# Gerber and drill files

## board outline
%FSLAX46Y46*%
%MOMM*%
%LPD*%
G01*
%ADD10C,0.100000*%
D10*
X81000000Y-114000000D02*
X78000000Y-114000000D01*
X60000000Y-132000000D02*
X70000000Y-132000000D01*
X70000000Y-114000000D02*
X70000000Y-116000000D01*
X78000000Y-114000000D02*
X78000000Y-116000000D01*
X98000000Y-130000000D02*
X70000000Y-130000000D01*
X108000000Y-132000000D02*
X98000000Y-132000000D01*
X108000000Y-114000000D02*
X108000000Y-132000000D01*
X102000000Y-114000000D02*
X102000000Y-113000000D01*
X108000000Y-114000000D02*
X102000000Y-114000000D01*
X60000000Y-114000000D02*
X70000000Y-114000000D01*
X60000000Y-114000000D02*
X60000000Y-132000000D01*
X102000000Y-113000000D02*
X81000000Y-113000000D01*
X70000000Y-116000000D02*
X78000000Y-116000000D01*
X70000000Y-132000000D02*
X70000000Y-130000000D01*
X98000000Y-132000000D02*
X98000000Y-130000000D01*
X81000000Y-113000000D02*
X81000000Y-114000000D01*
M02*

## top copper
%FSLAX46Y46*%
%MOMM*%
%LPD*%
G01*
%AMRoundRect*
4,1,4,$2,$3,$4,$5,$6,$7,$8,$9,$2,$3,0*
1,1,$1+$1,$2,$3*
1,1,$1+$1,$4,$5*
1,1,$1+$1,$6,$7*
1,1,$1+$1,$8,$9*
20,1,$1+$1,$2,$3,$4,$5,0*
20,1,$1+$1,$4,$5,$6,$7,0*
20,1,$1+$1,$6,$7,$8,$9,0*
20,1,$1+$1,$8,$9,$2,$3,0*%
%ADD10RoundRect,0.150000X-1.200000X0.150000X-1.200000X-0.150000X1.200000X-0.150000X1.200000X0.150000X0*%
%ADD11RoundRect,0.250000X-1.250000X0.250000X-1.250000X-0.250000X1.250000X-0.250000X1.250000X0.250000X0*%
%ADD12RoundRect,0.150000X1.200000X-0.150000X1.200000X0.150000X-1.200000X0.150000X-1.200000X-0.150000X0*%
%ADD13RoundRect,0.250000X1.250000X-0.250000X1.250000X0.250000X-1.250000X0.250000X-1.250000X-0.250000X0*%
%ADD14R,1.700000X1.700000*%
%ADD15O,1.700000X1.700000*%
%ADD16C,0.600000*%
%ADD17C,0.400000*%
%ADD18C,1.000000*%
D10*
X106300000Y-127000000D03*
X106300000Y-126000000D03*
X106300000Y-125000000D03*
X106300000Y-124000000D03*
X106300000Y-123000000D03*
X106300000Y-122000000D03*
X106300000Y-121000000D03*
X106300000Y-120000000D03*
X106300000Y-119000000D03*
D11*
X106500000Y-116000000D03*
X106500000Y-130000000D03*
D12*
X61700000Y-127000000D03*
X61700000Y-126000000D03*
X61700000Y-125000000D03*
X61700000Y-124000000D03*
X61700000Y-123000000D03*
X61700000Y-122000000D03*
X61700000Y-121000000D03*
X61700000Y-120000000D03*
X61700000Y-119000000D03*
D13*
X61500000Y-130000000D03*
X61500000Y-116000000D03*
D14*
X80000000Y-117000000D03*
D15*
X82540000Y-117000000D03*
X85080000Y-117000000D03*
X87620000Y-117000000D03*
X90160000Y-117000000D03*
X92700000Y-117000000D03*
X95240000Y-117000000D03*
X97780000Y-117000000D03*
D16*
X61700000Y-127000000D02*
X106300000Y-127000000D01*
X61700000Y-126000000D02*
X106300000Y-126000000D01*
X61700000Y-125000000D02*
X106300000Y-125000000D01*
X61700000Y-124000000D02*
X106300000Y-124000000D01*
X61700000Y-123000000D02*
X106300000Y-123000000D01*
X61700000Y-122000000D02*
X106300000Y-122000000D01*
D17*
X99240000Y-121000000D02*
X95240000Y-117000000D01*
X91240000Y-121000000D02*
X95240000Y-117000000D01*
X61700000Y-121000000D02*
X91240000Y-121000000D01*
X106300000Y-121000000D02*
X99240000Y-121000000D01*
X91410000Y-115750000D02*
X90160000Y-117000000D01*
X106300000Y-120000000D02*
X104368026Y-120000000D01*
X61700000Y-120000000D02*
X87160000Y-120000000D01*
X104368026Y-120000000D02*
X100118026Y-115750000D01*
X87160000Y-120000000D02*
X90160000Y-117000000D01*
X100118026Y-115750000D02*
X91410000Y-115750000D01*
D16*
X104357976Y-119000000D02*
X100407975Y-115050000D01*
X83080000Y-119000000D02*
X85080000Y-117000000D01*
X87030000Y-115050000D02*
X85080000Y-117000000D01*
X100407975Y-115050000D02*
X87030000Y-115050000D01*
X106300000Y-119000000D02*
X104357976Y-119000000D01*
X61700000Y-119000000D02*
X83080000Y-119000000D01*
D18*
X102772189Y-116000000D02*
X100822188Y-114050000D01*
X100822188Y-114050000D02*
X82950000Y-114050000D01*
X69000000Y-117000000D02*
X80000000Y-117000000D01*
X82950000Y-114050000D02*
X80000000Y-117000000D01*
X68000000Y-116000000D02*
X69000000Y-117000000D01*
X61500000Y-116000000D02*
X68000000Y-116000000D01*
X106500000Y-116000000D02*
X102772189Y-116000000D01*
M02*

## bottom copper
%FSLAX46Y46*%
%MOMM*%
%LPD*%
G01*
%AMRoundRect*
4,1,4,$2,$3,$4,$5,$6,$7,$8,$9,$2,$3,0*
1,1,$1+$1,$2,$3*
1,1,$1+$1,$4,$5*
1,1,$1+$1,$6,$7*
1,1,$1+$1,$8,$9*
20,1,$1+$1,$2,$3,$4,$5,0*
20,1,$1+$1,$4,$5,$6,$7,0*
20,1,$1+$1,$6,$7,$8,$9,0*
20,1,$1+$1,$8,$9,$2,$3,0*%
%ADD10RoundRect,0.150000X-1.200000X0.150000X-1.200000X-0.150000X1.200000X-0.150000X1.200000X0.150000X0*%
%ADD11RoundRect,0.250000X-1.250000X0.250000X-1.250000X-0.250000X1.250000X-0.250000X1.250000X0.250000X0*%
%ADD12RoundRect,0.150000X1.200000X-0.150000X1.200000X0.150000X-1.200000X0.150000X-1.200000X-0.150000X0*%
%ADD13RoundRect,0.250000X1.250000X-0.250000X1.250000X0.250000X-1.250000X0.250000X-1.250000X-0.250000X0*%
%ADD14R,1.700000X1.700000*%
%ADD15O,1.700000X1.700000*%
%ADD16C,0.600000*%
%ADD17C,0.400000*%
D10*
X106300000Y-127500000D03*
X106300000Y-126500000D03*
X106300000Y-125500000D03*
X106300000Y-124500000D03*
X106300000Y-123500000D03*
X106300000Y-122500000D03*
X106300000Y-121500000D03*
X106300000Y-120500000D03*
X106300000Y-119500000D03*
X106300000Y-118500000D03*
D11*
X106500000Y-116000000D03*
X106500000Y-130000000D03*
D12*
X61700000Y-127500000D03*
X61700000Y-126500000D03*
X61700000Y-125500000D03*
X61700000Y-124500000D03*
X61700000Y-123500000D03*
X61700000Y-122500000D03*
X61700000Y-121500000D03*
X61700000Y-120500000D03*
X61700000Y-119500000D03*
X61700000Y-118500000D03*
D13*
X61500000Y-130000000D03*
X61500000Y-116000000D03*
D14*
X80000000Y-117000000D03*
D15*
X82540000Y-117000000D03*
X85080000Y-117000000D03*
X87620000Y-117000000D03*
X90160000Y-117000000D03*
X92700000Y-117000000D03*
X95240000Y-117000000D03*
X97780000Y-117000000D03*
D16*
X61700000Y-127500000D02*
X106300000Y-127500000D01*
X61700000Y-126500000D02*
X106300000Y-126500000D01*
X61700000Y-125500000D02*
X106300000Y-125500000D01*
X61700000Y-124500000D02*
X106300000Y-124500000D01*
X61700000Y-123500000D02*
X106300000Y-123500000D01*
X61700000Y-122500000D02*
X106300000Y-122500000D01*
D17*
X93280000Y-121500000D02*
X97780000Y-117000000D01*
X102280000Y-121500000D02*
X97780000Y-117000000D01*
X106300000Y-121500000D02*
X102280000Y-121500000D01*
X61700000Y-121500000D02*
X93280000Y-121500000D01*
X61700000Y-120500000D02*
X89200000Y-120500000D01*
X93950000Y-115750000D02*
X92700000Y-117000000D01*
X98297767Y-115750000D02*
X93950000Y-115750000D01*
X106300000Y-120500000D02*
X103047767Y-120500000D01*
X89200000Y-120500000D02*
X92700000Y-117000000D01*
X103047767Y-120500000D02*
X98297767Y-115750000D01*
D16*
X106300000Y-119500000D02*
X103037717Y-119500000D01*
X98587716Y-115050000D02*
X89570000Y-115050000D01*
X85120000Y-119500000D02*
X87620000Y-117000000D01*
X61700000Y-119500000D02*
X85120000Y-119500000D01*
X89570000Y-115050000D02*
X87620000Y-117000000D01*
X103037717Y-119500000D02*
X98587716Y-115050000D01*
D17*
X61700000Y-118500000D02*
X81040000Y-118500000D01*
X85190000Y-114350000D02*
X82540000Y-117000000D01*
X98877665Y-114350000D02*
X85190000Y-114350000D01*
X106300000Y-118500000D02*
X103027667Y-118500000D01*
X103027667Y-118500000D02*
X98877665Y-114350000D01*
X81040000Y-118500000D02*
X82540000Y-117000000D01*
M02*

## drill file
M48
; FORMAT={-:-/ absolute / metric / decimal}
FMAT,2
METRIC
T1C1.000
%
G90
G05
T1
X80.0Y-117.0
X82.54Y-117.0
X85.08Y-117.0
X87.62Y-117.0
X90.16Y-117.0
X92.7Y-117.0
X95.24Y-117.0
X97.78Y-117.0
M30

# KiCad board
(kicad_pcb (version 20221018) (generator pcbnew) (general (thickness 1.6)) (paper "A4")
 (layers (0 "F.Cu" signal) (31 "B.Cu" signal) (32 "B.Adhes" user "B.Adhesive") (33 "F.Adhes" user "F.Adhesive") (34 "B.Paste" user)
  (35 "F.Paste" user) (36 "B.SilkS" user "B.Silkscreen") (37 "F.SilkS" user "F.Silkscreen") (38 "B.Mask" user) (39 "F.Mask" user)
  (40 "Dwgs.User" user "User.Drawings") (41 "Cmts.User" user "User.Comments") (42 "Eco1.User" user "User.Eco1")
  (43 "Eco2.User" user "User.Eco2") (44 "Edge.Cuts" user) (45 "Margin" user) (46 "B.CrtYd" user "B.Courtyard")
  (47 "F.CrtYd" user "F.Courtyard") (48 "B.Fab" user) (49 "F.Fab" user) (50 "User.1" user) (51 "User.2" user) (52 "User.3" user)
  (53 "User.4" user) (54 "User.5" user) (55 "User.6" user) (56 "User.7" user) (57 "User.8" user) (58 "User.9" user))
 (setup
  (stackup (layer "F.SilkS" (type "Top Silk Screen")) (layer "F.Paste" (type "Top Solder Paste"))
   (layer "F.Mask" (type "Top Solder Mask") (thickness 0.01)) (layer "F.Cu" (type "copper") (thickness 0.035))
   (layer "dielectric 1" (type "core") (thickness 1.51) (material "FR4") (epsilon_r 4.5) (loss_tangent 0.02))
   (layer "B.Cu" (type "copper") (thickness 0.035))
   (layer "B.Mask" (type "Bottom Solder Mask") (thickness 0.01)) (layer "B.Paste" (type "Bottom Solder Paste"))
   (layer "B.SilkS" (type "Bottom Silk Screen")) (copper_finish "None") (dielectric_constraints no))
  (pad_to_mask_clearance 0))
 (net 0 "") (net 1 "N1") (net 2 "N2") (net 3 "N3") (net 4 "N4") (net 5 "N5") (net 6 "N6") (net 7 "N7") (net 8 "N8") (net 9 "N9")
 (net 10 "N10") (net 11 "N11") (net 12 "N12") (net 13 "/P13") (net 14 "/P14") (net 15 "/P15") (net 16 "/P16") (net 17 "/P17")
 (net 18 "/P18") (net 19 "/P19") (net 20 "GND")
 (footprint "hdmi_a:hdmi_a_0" (layer "F.Cu") (at 108 123 -90)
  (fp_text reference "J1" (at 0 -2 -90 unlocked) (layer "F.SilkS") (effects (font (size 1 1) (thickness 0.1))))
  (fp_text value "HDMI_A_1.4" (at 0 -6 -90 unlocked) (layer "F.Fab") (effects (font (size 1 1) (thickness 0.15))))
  (pad "1" smd roundrect (at 4.5 1.7 270) (size 0.6 2.7) (layers "B.Cu" "B.Paste" "B.Mask") (roundrect_rratio 0.25) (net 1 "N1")
   (thermal_bridge_angle 45))
  (pad "2" smd roundrect (at 4 1.7 270) (size 0.6 2.7) (layers "F.Cu" "F.Paste" "F.Mask") (roundrect_rratio 0.25) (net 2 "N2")
   (thermal_bridge_angle 45))
  (pad "3" smd roundrect (at 3.5 1.7 270) (size 0.6 2.7) (layers "B.Cu" "B.Paste" "B.Mask") (roundrect_rratio 0.25) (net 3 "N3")
   (thermal_bridge_angle 45))
  (pad "4" smd roundrect (at 3 1.7 270) (size 0.6 2.7) (layers "F.Cu" "F.Paste" "F.Mask") (roundrect_rratio 0.25) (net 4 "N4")
   (thermal_bridge_angle 45))
  (pad "5" smd roundrect (at 2.5 1.7 270) (size 0.6 2.7) (layers "B.Cu" "B.Paste" "B.Mask") (roundrect_rratio 0.25) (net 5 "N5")
   (thermal_bridge_angle 45))
  (pad "6" smd roundrect (at 2 1.7 270) (size 0.6 2.7) (layers "F.Cu" "F.Paste" "F.Mask") (roundrect_rratio 0.25) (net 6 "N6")
   (thermal_bridge_angle 45))
  (pad "7" smd roundrect (at 1.5 1.7 270) (size 0.6 2.7) (layers "B.Cu" "B.Paste" "B.Mask") (roundrect_rratio 0.25) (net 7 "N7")
   (thermal_bridge_angle 45))
  (pad "8" smd roundrect (at 1 1.7 270) (size 0.6 2.7) (layers "F.Cu" "F.Paste" "F.Mask") (roundrect_rratio 0.25) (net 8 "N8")
   (thermal_bridge_angle 45))
  (pad "9" smd roundrect (at 0.5 1.7 270) (size 0.6 2.7) (layers "B.Cu" "B.Paste" "B.Mask") (roundrect_rratio 0.25) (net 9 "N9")
   (thermal_bridge_angle 45))
  (pad "10" smd roundrect (at 0 1.7 270) (size 0.6 2.7) (layers "F.Cu" "F.Paste" "F.Mask") (roundrect_rratio 0.25) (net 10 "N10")
   (thermal_bridge_angle 45))
  (pad "11" smd roundrect (at -0.5 1.7 270) (size 0.6 2.7) (layers "B.Cu" "B.Paste" "B.Mask") (roundrect_rratio 0.25) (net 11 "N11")
   (thermal_bridge_angle 45))
  (pad "12" smd roundrect (at -1 1.7 270) (size 0.6 2.7) (layers "F.Cu" "F.Paste" "F.Mask") (roundrect_rratio 0.25) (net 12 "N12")
   (thermal_bridge_angle 45))
  (pad "13" smd roundrect (at -1.5 1.7 270) (size 0.6 2.7) (layers "B.Cu" "B.Paste" "B.Mask") (roundrect_rratio 0.25) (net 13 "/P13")
   (thermal_bridge_angle 45))
  (pad "14" smd roundrect (at -2 1.7 270) (size 0.6 2.7) (layers "F.Cu" "F.Paste" "F.Mask") (roundrect_rratio 0.25) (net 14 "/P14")
   (thermal_bridge_angle 45))
  (pad "15" smd roundrect (at -2.5 1.7 270) (size 0.6 2.7) (layers "B.Cu" "B.Paste" "B.Mask") (roundrect_rratio 0.25) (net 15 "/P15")
   (thermal_bridge_angle 45))
  (pad "16" smd roundrect (at -3 1.7 270) (size 0.6 2.7) (layers "F.Cu" "F.Paste" "F.Mask") (roundrect_rratio 0.25) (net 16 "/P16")
   (thermal_bridge_angle 45))
  (pad "17" smd roundrect (at -3.5 1.7 270) (size 0.6 2.7) (layers "B.Cu" "B.Paste" "B.Mask") (roundrect_rratio 0.25) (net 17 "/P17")
   (thermal_bridge_angle 45))
  (pad "18" smd roundrect (at -4 1.7 270) (size 0.6 2.7) (layers "F.Cu" "F.Paste" "F.Mask") (roundrect_rratio 0.25) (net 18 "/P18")
   (thermal_bridge_angle 45))
  (pad "19" smd roundrect (at -4.5 1.7 270) (size 0.6 2.7) (layers "B.Cu" "B.Paste" "B.Mask") (roundrect_rratio 0.25) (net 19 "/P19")
   (thermal_bridge_angle 45))
  (pad "SH" smd roundrect (at -7 1.5 270) (size 1 3) (layers "F.Cu" "F.Paste" "F.Mask") (roundrect_rratio 0.25) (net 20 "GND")
   (thermal_bridge_angle 45))
  (pad "SH" smd roundrect (at -7 1.5 270) (size 1 3) (layers "B.Cu" "B.Paste" "B.Mask") (roundrect_rratio 0.25) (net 20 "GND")
   (thermal_bridge_angle 45))
  (pad "SH" smd roundrect (at 7 1.5 270) (size 1 3) (layers "F.Cu" "F.Paste" "F.Mask") (roundrect_rratio 0.25) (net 20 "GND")
   (thermal_bridge_angle 45))
  (pad "SH" smd roundrect (at 7 1.5 270) (size 1 3) (layers "B.Cu" "B.Paste" "B.Mask") (roundrect_rratio 0.25) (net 20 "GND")
   (thermal_bridge_angle 45)))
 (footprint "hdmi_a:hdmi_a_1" (layer "F.Cu") (at 60 123 90)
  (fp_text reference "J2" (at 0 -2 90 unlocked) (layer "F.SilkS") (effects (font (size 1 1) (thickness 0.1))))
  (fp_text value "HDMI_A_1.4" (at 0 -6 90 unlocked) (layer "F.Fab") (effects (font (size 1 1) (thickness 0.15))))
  (pad "1" smd roundrect (at -4.5 1.7 90) (size 0.6 2.7) (layers "B.Cu" "B.Paste" "B.Mask") (roundrect_rratio 0.25) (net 1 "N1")
   (thermal_bridge_angle 45))
  (pad "2" smd roundrect (at -4 1.7 90) (size 0.6 2.7) (layers "F.Cu" "F.Paste" "F.Mask") (roundrect_rratio 0.25) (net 2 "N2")
   (thermal_bridge_angle 45))
  (pad "3" smd roundrect (at -3.5 1.7 90) (size 0.6 2.7) (layers "B.Cu" "B.Paste" "B.Mask") (roundrect_rratio 0.25) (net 3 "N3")
   (thermal_bridge_angle 45))
  (pad "4" smd roundrect (at -3 1.7 90) (size 0.6 2.7) (layers "F.Cu" "F.Paste" "F.Mask") (roundrect_rratio 0.25) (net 4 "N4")
   (thermal_bridge_angle 45))
  (pad "5" smd roundrect (at -2.5 1.7 90) (size 0.6 2.7) (layers "B.Cu" "B.Paste" "B.Mask") (roundrect_rratio 0.25) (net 5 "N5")
   (thermal_bridge_angle 45))
  (pad "6" smd roundrect (at -2 1.7 90) (size 0.6 2.7) (layers "F.Cu" "F.Paste" "F.Mask") (roundrect_rratio 0.25) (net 6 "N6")
   (thermal_bridge_angle 45))
  (pad "7" smd roundrect (at -1.5 1.7 90) (size 0.6 2.7) (layers "B.Cu" "B.Paste" "B.Mask") (roundrect_rratio 0.25) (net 7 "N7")
   (thermal_bridge_angle 45))
  (pad "8" smd roundrect (at -1 1.7 90) (size 0.6 2.7) (layers "F.Cu" "F.Paste" "F.Mask") (roundrect_rratio 0.25) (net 8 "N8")
   (thermal_bridge_angle 45))
  (pad "9" smd roundrect (at -0.5 1.7 90) (size 0.6 2.7) (layers "B.Cu" "B.Paste" "B.Mask") (roundrect_rratio 0.25) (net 9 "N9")
   (thermal_bridge_angle 45))
  (pad "10" smd roundrect (at 0 1.7 90) (size 0.6 2.7) (layers "F.Cu" "F.Paste" "F.Mask") (roundrect_rratio 0.25) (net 10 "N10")
   (thermal_bridge_angle 45))
  (pad "11" smd roundrect (at 0.5 1.7 90) (size 0.6 2.7) (layers "B.Cu" "B.Paste" "B.Mask") (roundrect_rratio 0.25) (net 11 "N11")
   (thermal_bridge_angle 45))
  (pad "12" smd roundrect (at 1 1.7 90) (size 0.6 2.7) (layers "F.Cu" "F.Paste" "F.Mask") (roundrect_rratio 0.25) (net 12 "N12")
   (thermal_bridge_angle 45))
  (pad "13" smd roundrect (at 1.5 1.7 90) (size 0.6 2.7) (layers "B.Cu" "B.Paste" "B.Mask") (roundrect_rratio 0.25) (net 13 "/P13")
   (thermal_bridge_angle 45))
  (pad "14" smd roundrect (at 2 1.7 90) (size 0.6 2.7) (layers "F.Cu" "F.Paste" "F.Mask") (roundrect_rratio 0.25) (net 14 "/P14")
   (thermal_bridge_angle 45))
  (pad "15" smd roundrect (at 2.5 1.7 90) (size 0.6 2.7) (layers "B.Cu" "B.Paste" "B.Mask") (roundrect_rratio 0.25) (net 15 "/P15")
   (thermal_bridge_angle 45))
  (pad "16" smd roundrect (at 3 1.7 90) (size 0.6 2.7) (layers "F.Cu" "F.Paste" "F.Mask") (roundrect_rratio 0.25) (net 16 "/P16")
   (thermal_bridge_angle 45))
  (pad "17" smd roundrect (at 3.5 1.7 90) (size 0.6 2.7) (layers "B.Cu" "B.Paste" "B.Mask") (roundrect_rratio 0.25) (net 17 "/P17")
   (thermal_bridge_angle 45))
  (pad "18" smd roundrect (at 4 1.7 90) (size 0.6 2.7) (layers "F.Cu" "F.Paste" "F.Mask") (roundrect_rratio 0.25) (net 18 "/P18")
   (thermal_bridge_angle 45))
  (pad "19" smd roundrect (at 4.5 1.7 90) (size 0.6 2.7) (layers "B.Cu" "B.Paste" "B.Mask") (roundrect_rratio 0.25) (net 19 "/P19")
   (thermal_bridge_angle 45))
  (pad "SH" smd roundrect (at -7 1.5 90) (size 1 3) (layers "F.Cu" "F.Paste" "F.Mask") (roundrect_rratio 0.25) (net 20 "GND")
   (thermal_bridge_angle 45))
  (pad "SH" smd roundrect (at -7 1.5 90) (size 1 3) (layers "B.Cu" "B.Paste" "B.Mask") (roundrect_rratio 0.25) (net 20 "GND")
   (thermal_bridge_angle 45))
  (pad "SH" smd roundrect (at 7 1.5 90) (size 1 3) (layers "F.Cu" "F.Paste" "F.Mask") (roundrect_rratio 0.25) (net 20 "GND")
   (thermal_bridge_angle 45))
  (pad "SH" smd roundrect (at 7 1.5 90) (size 1 3) (layers "B.Cu" "B.Paste" "B.Mask") (roundrect_rratio 0.25) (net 20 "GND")
   (thermal_bridge_angle 45)))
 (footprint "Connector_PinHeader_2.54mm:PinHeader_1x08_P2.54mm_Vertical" (layer "B.Cu") (at 80 117 -90)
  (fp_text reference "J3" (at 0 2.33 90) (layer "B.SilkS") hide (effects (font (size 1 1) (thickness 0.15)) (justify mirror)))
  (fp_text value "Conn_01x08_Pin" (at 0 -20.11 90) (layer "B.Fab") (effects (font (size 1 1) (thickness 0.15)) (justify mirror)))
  (pad "1" thru_hole rect (at 0 0 270) (size 1.7 1.7) (drill 1) (layers "*.Cu" "*.Mask") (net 20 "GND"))
  (pad "2" thru_hole oval (at 0 -2.54 270) (size 1.7 1.7) (drill 1) (layers "*.Cu" "*.Mask") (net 19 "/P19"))
  (pad "3" thru_hole oval (at 0 -5.08 270) (size 1.7 1.7) (drill 1) (layers "*.Cu" "*.Mask") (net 18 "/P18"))
  (pad "4" thru_hole oval (at 0 -7.62 270) (size 1.7 1.7) (drill 1) (layers "*.Cu" "*.Mask") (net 17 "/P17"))
  (pad "5" thru_hole oval (at 0 -10.16 270) (size 1.7 1.7) (drill 1) (layers "*.Cu" "*.Mask") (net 16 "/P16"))
  (pad "6" thru_hole oval (at 0 -12.7 270) (size 1.7 1.7) (drill 1) (layers "*.Cu" "*.Mask") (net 15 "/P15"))
  (pad "7" thru_hole oval (at 0 -15.24 270) (size 1.7 1.7) (drill 1) (layers "*.Cu" "*.Mask") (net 14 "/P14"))
  (pad "8" thru_hole oval (at 0 -17.78 270) (size 1.7 1.7) (drill 1) (layers "*.Cu" "*.Mask") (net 13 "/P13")))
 (gr_line (start 81 114) (end 78 114) (stroke (width 0.1) (type default)) (layer "Edge.Cuts"))
 (gr_line (start 60 132) (end 70 132) (stroke (width 0.1) (type default)) (layer "Edge.Cuts"))
 (gr_line (start 70 114) (end 70 116) (stroke (width 0.1) (type default)) (layer "Edge.Cuts"))
 (gr_line (start 78 114) (end 78 116) (stroke (width 0.1) (type default)) (layer "Edge.Cuts"))
 (gr_line (start 98 130) (end 70 130) (stroke (width 0.1) (type default)) (layer "Edge.Cuts"))
 (gr_line (start 108 132) (end 98 132) (stroke (width 0.1) (type default)) (layer "Edge.Cuts"))
 (gr_line (start 108 114) (end 108 132) (stroke (width 0.1) (type default)) (layer "Edge.Cuts"))
 (gr_line (start 102 114) (end 102 113) (stroke (width 0.1) (type default)) (layer "Edge.Cuts"))
 (gr_line (start 108 114) (end 102 114) (stroke (width 0.1) (type default)) (layer "Edge.Cuts"))
 (gr_line (start 60 114) (end 70 114) (stroke (width 0.1) (type default)) (layer "Edge.Cuts"))
 (gr_line (start 60 114) (end 60 132) (stroke (width 0.1) (type default)) (layer "Edge.Cuts"))
 (gr_line (start 102 113) (end 81 113) (stroke (width 0.1) (type default)) (layer "Edge.Cuts"))
 (gr_line (start 70 116) (end 78 116) (stroke (width 0.1) (type default)) (layer "Edge.Cuts"))
 (gr_line (start 70 132) (end 70 130) (stroke (width 0.1) (type default)) (layer "Edge.Cuts"))
 (gr_line (start 98 132) (end 98 130) (stroke (width 0.1) (type default)) (layer "Edge.Cuts"))
 (gr_line (start 81 113) (end 81 114) (stroke (width 0.1) (type default)) (layer "Edge.Cuts"))
 (segment (start 61.7 127.5) (end 106.3 127.5) (width 0.6) (layer "B.Cu") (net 1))
 (segment (start 61.7 127) (end 106.3 127) (width 0.6) (layer "F.Cu") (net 2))
 (segment (start 61.7 126.5) (end 106.3 126.5) (width 0.6) (layer "B.Cu") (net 3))
 (segment (start 61.7 126) (end 106.3 126) (width 0.6) (layer "F.Cu") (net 4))
 (segment (start 61.7 125.5) (end 106.3 125.5) (width 0.6) (layer "B.Cu") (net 5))
 (segment (start 61.7 125) (end 106.3 125) (width 0.6) (layer "F.Cu") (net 6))
 (segment (start 61.7 124.5) (end 106.3 124.5) (width 0.6) (layer "B.Cu") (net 7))
 (segment (start 61.7 124) (end 106.3 124) (width 0.6) (layer "F.Cu") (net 8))
 (segment (start 61.7 123.5) (end 106.3 123.5) (width 0.6) (layer "B.Cu") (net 9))
 (segment (start 61.7 123) (end 106.3 123) (width 0.6) (layer "F.Cu") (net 10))
 (segment (start 61.7 122.5) (end 106.3 122.5) (width 0.6) (layer "B.Cu") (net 11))
 (segment (start 61.7 122) (end 106.3 122) (width 0.6) (layer "F.Cu") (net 12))
 (segment (start 93.28 121.5) (end 97.78 117) (width 0.4) (layer "B.Cu") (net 13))
 (segment (start 102.28 121.5) (end 97.78 117) (width 0.4) (layer "B.Cu") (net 13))
 (segment (start 106.3 121.5) (end 102.28 121.5) (width 0.4) (layer "B.Cu") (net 13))
 (segment (start 61.7 121.5) (end 93.28 121.5) (width 0.4) (layer "B.Cu") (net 13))
 (segment (start 99.24 121) (end 95.24 117) (width 0.4) (layer "F.Cu") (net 14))
 (segment (start 91.24 121) (end 95.24 117) (width 0.4) (layer "F.Cu") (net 14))
 (segment (start 61.7 121) (end 91.24 121) (width 0.4) (layer "F.Cu") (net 14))
 (segment (start 106.3 121) (end 99.24 121) (width 0.4) (layer "F.Cu") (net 14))
 (segment (start 61.7 120.5) (end 89.2 120.5) (width 0.4) (layer "B.Cu") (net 15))
 (segment (start 93.95 115.75) (end 92.7 117) (width 0.4) (layer "B.Cu") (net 15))
 (segment (start 98.297767 115.75) (end 93.95 115.75) (width 0.4) (layer "B.Cu") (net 15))
 (segment (start 106.3 120.5) (end 103.047767 120.5) (width 0.4) (layer "B.Cu") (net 15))
 (segment (start 89.2 120.5) (end 92.7 117) (width 0.4) (layer "B.Cu") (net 15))
 (segment (start 103.047767 120.5) (end 98.297767 115.75) (width 0.4) (layer "B.Cu") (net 15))
 (segment (start 91.41 115.75) (end 90.16 117) (width 0.4) (layer "F.Cu") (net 16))
 (segment (start 106.3 120) (end 104.368026 120) (width 0.4) (layer "F.Cu") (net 16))
 (segment (start 61.7 120) (end 87.16 120) (width 0.4) (layer "F.Cu") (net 16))
 (segment (start 104.368026 120) (end 100.118026 115.75) (width 0.4) (layer "F.Cu") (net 16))
 (segment (start 87.16 120) (end 90.16 117) (width 0.4) (layer "F.Cu") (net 16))
 (segment (start 100.118026 115.75) (end 91.41 115.75) (width 0.4) (layer "F.Cu") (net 16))
 (segment (start 106.3 119.5) (end 103.037717 119.5) (width 0.6) (layer "B.Cu") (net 17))
 (segment (start 98.587716 115.05) (end 89.57 115.05) (width 0.6) (layer "B.Cu") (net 17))
 (segment (start 85.12 119.5) (end 87.62 117) (width 0.6) (layer "B.Cu") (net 17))
 (segment (start 61.7 119.5) (end 85.12 119.5) (width 0.6) (layer "B.Cu") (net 17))
 (segment (start 89.57 115.05) (end 87.62 117) (width 0.6) (layer "B.Cu") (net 17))
 (segment (start 103.037717 119.5) (end 98.587716 115.05) (width 0.6) (layer "B.Cu") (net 17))
 (segment (start 104.357976 119) (end 100.407975 115.05) (width 0.6) (layer "F.Cu") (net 18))
 (segment (start 83.08 119) (end 85.08 117) (width 0.6) (layer "F.Cu") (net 18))
 (segment (start 87.03 115.05) (end 85.08 117) (width 0.6) (layer "F.Cu") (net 18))
 (segment (start 100.407975 115.05) (end 87.03 115.05) (width 0.6) (layer "F.Cu") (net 18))
 (segment (start 106.3 119) (end 104.357976 119) (width 0.6) (layer "F.Cu") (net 18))
 (segment (start 61.7 119) (end 83.08 119) (width 0.6) (layer "F.Cu") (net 18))
 (segment (start 61.7 118.5) (end 81.04 118.5) (width 0.4) (layer "B.Cu") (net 19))
 (segment (start 85.19 114.35) (end 82.54 117) (width 0.4) (layer "B.Cu") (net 19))
 (segment (start 98.877665 114.35) (end 85.19 114.35) (width 0.4) (layer "B.Cu") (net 19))
 (segment (start 106.3 118.5) (end 103.027667 118.5) (width 0.4) (layer "B.Cu") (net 19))
 (segment (start 103.027667 118.5) (end 98.877665 114.35) (width 0.4) (layer "B.Cu") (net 19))
 (segment (start 81.04 118.5) (end 82.54 117) (width 0.4) (layer "B.Cu") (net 19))
 (segment (start 102.772189 116) (end 100.822188 114.05) (width 1) (layer "F.Cu") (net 20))
 (segment (start 100.822188 114.05) (end 82.95 114.05) (width 1) (layer "F.Cu") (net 20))
 (segment (start 69 117) (end 80 117) (width 1) (layer "F.Cu") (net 20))
 (segment (start 82.95 114.05) (end 80 117) (width 1) (layer "F.Cu") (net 20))
 (segment (start 68 116) (end 69 117) (width 1) (layer "F.Cu") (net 20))
 (segment (start 61.5 116) (end 68 116) (width 1) (layer "F.Cu") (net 20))
 (segment (start 106.5 116) (end 102.772189 116) (width 1) (layer "F.Cu") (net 20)))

